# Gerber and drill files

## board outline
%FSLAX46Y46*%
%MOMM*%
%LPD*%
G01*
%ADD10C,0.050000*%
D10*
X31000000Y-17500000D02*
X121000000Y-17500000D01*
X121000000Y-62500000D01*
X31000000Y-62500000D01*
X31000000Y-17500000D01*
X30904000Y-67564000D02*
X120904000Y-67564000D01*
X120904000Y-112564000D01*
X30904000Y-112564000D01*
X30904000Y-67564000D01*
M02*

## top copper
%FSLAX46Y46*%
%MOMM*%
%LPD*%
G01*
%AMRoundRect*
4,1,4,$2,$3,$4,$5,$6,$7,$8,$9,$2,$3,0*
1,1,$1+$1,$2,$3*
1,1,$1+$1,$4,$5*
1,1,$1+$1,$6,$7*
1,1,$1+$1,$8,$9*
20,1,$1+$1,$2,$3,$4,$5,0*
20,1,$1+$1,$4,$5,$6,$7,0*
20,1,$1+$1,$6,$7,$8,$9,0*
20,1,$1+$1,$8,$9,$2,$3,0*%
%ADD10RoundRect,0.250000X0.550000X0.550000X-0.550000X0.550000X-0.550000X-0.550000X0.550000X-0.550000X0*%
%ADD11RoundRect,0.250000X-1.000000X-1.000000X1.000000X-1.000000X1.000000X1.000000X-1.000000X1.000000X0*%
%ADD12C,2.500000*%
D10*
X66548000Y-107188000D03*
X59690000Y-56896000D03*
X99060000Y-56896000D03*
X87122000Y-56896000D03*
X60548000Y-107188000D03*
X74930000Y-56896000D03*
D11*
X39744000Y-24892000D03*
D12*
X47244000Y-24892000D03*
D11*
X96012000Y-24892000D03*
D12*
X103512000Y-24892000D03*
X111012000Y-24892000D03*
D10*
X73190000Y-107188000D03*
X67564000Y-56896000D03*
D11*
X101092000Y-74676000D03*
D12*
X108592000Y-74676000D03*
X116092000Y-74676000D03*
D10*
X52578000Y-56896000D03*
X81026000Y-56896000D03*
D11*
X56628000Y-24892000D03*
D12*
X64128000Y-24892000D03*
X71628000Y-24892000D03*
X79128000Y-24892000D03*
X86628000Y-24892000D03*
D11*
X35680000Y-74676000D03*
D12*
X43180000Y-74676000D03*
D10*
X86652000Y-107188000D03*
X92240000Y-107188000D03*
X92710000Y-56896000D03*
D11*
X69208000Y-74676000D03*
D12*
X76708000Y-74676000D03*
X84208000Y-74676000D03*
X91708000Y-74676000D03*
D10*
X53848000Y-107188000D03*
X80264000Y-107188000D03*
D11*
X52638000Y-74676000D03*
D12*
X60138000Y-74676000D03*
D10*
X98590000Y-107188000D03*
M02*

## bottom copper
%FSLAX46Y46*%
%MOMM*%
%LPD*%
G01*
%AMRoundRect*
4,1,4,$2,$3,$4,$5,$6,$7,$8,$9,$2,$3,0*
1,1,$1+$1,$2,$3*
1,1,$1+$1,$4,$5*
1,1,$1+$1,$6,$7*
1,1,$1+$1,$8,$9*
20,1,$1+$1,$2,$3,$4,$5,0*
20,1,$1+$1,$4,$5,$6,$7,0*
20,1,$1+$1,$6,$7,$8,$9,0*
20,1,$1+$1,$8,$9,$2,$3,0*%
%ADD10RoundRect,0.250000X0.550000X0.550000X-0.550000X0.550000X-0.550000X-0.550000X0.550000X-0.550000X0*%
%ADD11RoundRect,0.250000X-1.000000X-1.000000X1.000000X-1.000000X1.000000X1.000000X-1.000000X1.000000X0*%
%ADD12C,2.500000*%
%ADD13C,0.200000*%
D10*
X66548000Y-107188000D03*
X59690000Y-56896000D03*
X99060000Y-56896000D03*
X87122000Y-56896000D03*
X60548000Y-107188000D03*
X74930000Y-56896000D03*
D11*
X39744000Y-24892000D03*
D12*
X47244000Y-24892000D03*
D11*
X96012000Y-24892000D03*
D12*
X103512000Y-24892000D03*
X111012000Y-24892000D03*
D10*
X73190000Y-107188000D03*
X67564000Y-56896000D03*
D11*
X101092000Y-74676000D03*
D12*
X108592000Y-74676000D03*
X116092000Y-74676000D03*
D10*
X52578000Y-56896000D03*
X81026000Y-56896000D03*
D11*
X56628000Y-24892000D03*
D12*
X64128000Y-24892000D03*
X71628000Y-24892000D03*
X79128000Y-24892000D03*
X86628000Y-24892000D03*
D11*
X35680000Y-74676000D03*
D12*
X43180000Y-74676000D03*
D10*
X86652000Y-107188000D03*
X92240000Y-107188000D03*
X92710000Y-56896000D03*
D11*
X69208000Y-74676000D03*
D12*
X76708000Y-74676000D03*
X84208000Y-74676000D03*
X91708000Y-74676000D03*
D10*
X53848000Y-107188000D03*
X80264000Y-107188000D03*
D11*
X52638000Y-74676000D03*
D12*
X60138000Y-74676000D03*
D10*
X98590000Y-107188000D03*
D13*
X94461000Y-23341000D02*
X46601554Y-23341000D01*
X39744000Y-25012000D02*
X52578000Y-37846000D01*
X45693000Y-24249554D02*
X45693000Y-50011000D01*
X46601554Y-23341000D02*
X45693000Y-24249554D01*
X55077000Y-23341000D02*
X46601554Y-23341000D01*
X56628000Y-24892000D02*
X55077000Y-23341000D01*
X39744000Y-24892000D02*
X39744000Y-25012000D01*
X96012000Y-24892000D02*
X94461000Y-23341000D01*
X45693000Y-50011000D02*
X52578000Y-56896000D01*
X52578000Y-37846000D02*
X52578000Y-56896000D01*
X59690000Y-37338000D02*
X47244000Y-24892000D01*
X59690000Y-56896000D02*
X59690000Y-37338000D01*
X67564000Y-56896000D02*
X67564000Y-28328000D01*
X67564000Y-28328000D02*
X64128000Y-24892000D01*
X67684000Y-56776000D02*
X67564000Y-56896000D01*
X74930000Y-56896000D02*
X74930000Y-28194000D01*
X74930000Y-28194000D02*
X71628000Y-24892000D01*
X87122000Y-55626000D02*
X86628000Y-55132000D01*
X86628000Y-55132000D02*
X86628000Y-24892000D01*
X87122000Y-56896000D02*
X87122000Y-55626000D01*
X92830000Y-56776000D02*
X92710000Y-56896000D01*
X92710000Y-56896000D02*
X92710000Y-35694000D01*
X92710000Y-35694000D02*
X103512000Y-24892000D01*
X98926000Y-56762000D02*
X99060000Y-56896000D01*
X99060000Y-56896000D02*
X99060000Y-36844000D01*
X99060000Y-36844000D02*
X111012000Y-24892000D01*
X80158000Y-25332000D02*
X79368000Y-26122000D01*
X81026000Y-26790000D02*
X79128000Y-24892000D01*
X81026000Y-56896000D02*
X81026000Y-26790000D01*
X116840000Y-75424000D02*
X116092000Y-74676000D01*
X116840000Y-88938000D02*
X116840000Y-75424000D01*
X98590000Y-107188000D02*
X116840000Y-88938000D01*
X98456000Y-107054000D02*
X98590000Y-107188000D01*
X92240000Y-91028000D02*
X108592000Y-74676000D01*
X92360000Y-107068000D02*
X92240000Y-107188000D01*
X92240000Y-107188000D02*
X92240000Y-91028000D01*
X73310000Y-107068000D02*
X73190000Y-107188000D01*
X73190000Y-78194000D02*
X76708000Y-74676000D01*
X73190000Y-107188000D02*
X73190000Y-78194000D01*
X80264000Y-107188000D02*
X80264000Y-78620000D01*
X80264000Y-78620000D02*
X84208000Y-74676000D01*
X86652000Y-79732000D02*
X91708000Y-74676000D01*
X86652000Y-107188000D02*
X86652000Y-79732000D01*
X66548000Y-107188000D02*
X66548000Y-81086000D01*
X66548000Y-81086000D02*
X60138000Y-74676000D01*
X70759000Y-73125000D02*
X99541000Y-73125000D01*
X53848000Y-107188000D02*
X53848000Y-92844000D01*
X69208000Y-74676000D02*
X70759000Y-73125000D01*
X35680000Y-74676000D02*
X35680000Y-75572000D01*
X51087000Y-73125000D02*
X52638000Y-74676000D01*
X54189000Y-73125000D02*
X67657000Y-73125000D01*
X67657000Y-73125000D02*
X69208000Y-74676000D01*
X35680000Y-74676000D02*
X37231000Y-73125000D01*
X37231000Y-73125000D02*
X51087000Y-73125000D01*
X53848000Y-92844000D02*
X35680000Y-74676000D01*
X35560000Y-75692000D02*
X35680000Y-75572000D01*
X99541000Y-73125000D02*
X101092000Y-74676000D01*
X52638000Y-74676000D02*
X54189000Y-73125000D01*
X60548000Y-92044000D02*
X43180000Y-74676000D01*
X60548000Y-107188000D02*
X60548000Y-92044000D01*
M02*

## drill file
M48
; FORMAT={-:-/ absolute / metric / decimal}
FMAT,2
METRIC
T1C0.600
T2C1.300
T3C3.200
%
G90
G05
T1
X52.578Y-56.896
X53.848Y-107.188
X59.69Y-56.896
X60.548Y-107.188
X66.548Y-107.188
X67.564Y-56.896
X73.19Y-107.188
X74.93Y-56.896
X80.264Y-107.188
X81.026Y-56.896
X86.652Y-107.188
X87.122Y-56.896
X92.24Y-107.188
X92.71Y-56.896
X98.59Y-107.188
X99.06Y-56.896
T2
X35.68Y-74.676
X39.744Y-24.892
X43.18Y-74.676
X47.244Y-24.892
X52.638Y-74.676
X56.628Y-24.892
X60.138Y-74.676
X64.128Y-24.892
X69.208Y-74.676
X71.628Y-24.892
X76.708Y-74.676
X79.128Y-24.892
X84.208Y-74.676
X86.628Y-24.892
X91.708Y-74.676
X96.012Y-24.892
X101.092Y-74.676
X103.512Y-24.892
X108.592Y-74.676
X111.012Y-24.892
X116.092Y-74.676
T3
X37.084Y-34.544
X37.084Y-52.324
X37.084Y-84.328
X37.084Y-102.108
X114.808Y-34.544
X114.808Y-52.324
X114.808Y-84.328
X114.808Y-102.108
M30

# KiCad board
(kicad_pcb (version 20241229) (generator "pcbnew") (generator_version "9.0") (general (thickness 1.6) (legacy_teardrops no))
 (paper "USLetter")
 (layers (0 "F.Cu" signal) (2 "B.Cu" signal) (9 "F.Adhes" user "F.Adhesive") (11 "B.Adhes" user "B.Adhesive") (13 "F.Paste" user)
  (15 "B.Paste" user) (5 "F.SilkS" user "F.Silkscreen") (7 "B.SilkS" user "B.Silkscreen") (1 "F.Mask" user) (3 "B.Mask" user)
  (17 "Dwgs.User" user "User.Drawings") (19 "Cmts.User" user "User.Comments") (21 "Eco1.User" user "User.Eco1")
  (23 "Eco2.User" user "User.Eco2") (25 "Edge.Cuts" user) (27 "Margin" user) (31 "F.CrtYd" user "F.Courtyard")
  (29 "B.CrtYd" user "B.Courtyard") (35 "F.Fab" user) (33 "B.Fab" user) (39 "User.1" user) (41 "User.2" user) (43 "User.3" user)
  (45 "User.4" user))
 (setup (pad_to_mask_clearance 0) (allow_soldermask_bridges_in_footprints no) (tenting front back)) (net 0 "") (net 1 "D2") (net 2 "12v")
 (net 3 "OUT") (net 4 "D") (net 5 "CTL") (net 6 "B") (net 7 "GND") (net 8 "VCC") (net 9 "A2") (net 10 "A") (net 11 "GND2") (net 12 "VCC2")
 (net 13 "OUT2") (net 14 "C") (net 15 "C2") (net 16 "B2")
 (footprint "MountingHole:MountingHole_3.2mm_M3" (layer "F.Cu") (at 114.808 102.108)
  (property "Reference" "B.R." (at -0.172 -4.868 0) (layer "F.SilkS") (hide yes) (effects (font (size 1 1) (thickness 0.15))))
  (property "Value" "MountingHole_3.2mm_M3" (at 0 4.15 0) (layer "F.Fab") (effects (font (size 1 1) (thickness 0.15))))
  (pad "" np_thru_hole circle (at 0 0) (size 3.2 3.2) (drill 3.2) (layers "*.Cu" "*.Mask")))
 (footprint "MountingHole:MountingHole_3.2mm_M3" (layer "F.Cu") (at 114.808 52.324)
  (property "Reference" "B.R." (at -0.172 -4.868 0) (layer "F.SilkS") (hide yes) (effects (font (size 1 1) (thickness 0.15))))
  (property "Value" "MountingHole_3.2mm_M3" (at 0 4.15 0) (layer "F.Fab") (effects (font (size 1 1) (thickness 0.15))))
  (pad "" np_thru_hole circle (at 0 0) (size 3.2 3.2) (drill 3.2) (layers "*.Cu" "*.Mask")))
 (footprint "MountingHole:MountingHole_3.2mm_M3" (layer "F.Cu") (at 37.084 102.108)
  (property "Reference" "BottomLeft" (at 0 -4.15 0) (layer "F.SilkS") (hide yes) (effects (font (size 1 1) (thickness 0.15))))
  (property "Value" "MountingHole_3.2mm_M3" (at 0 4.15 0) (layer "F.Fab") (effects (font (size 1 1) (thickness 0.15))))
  (pad "" np_thru_hole circle (at 0 0) (size 3.2 3.2) (drill 3.2) (layers "*.Cu" "*.Mask")))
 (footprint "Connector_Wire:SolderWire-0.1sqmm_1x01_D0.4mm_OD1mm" (layer "F.Cu") (at 66.548 107.188 180)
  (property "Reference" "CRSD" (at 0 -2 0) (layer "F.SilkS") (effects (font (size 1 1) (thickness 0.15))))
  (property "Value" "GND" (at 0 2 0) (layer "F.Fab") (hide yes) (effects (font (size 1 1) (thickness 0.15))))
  (pad "1" thru_hole roundrect (at 0 0 180) (size 1.6 1.6) (drill 0.6) (layers "*.Cu" "*.Mask") (remove_unused_layers no)
   (roundrect_rratio 0.15625) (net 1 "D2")))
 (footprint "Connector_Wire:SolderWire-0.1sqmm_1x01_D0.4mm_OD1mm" (layer "F.Cu") (at 59.69 56.896 180)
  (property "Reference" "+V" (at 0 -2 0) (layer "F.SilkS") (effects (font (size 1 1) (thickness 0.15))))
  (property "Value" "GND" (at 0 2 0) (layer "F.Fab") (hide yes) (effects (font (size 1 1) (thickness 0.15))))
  (pad "1" thru_hole roundrect (at 0 0 180) (size 1.6 1.6) (drill 0.6) (layers "*.Cu" "*.Mask") (remove_unused_layers no)
   (roundrect_rratio 0.15625) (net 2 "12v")))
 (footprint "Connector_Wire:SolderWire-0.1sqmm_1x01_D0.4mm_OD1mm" (layer "F.Cu") (at 99.06 56.896 180)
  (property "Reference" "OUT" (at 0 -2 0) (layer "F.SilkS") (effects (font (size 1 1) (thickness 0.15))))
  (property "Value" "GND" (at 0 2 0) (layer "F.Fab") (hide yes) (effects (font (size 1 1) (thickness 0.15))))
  (pad "1" thru_hole roundrect (at 0 0 180) (size 1.6 1.6) (drill 0.6) (layers "*.Cu" "*.Mask") (remove_unused_layers no)
   (roundrect_rratio 0.15625) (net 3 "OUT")))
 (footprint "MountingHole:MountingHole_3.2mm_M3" (layer "F.Cu") (at 114.808 84.328)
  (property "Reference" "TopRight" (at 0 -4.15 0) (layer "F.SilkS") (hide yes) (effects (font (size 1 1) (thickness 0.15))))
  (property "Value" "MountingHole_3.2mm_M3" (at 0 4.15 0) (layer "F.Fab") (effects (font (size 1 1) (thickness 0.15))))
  (pad "" np_thru_hole circle (at 0 0) (size 3.2 3.2) (drill 3.2) (layers "*.Cu" "*.Mask")))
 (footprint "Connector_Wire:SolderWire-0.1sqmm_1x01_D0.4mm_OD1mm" (layer "F.Cu") (at 87.122 56.896 180)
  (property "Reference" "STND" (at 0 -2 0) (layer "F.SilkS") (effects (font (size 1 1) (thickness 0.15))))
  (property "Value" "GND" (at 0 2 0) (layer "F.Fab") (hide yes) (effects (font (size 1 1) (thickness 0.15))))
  (pad "1" thru_hole roundrect (at 0 0 180) (size 1.6 1.6) (drill 0.6) (layers "*.Cu" "*.Mask") (remove_unused_layers no)
   (roundrect_rratio 0.15625) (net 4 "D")))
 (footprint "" (layer "F.Cu") (at 60.548 107.188)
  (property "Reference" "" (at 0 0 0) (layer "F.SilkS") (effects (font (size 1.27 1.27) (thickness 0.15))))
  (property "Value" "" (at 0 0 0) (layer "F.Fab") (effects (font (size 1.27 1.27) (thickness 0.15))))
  (pad "1" thru_hole roundrect (at 0 0 180) (size 1.6 1.6) (drill 0.6) (layers "*.Cu" "*.Mask") (remove_unused_layers no)
   (roundrect_rratio 0.15625) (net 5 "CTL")))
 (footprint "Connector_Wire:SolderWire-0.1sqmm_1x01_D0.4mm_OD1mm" (layer "F.Cu") (at 74.93 56.896 180)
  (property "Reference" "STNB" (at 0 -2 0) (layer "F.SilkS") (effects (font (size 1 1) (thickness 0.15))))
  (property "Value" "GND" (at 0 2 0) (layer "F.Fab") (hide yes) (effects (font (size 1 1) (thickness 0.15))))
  (pad "1" thru_hole roundrect (at 0 0 180) (size 1.6 1.6) (drill 0.6) (layers "*.Cu" "*.Mask") (remove_unused_layers no)
   (roundrect_rratio 0.15625) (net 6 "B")))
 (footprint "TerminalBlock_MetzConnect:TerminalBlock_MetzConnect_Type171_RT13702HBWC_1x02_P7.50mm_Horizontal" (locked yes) (layer "F.Cu")
  (at 39.744 24.892)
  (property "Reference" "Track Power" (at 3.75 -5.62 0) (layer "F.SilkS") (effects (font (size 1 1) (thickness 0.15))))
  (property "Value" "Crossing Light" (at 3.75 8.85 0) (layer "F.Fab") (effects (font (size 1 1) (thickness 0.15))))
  (pad "1" thru_hole roundrect (at 0 0) (size 2.5 2.5) (drill 1.3) (layers "*.Cu" "*.Mask") (remove_unused_layers no) (roundrect_rratio 0.1)
   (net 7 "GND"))
  (pad "2" thru_hole circle (at 7.5 0) (size 2.5 2.5) (drill 1.3) (layers "*.Cu" "*.Mask") (remove_unused_layers no) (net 2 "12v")))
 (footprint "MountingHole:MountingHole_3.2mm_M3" (layer "F.Cu") (at 37.084 34.544)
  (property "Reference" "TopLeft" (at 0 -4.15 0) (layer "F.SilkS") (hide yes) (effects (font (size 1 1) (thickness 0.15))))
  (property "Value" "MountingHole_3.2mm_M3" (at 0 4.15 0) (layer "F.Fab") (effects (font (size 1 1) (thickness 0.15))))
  (pad "" np_thru_hole circle (at 0 0) (size 3.2 3.2) (drill 3.2) (layers "*.Cu" "*.Mask")))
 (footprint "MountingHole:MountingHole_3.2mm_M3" (layer "F.Cu") (at 37.084 52.324)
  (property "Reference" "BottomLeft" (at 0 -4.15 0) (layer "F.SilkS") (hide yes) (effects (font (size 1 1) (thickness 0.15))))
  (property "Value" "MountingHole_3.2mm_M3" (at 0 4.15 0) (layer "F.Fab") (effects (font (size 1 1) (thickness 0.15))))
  (pad "" np_thru_hole circle (at 0 0) (size 3.2 3.2) (drill 3.2) (layers "*.Cu" "*.Mask")))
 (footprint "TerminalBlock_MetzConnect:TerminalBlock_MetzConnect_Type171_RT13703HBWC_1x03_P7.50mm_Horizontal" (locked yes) (layer "F.Cu")
  (at 96.012 24.892)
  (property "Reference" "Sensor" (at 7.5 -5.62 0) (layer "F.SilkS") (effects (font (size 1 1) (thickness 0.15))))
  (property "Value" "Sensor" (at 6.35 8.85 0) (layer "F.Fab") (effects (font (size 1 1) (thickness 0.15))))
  (pad "1" thru_hole roundrect (at 0 0) (size 2.5 2.5) (drill 1.3) (layers "*.Cu" "*.Mask") (remove_unused_layers no) (roundrect_rratio 0.1)
   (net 7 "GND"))
  (pad "2" thru_hole circle (at 7.5 0) (size 2.5 2.5) (drill 1.3) (layers "*.Cu" "*.Mask") (remove_unused_layers no) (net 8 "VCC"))
  (pad "3" thru_hole circle (at 15 0) (size 2.5 2.5) (drill 1.3) (layers "*.Cu" "*.Mask") (remove_unused_layers no) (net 3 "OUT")))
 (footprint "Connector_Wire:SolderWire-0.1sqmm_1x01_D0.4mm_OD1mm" (layer "F.Cu") (at 73.19 107.188 180)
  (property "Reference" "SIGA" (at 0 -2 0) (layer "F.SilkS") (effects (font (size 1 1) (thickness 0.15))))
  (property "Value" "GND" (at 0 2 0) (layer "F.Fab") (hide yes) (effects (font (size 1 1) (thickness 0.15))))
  (pad "1" thru_hole roundrect (at 0 0 180) (size 1.6 1.6) (drill 0.6) (layers "*.Cu" "*.Mask") (remove_unused_layers no)
   (roundrect_rratio 0.15625) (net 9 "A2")))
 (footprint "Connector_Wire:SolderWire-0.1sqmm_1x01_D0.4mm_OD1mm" (layer "F.Cu") (at 67.564 56.896 180)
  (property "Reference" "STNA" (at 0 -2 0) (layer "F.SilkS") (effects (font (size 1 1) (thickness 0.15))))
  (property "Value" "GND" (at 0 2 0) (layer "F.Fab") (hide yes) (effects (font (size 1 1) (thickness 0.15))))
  (pad "1" thru_hole roundrect (at 0 0 180) (size 1.6 1.6) (drill 0.6) (layers "*.Cu" "*.Mask") (remove_unused_layers no)
   (roundrect_rratio 0.15625) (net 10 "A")))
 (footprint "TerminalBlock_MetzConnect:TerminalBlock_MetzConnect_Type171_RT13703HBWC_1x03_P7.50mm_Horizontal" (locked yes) (layer "F.Cu")
  (at 101.092 74.676)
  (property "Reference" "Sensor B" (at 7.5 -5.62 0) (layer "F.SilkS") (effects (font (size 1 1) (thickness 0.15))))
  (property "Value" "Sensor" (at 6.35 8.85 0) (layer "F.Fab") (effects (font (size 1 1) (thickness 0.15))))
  (pad "1" thru_hole roundrect (at 0 0) (size 2.5 2.5) (drill 1.3) (layers "*.Cu" "*.Mask") (remove_unused_layers no) (roundrect_rratio 0.1)
   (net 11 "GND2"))
  (pad "2" thru_hole circle (at 7.5 0) (size 2.5 2.5) (drill 1.3) (layers "*.Cu" "*.Mask") (remove_unused_layers no) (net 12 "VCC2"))
  (pad "3" thru_hole circle (at 15 0) (size 2.5 2.5) (drill 1.3) (layers "*.Cu" "*.Mask") (remove_unused_layers no) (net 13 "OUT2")))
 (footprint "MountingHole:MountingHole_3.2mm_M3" (layer "F.Cu") (at 114.808 34.544)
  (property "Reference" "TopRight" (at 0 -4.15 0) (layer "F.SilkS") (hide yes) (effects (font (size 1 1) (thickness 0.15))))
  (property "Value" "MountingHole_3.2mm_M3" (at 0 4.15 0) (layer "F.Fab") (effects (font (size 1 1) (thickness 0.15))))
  (pad "" np_thru_hole circle (at 0 0) (size 3.2 3.2) (drill 3.2) (layers "*.Cu" "*.Mask")))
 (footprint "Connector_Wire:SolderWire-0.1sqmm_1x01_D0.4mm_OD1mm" (layer "F.Cu") (at 52.578 56.896 180)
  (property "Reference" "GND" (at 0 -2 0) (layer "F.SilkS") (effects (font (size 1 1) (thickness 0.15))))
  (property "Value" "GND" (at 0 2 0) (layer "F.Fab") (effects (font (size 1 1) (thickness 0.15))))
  (pad "1" thru_hole roundrect (at 0 0 180) (size 1.6 1.6) (drill 0.6) (layers "*.Cu" "*.Mask") (remove_unused_layers no)
   (roundrect_rratio 0.15625) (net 7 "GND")))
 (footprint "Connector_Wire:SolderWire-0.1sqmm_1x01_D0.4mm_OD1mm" (layer "F.Cu") (at 81.026 56.896 180)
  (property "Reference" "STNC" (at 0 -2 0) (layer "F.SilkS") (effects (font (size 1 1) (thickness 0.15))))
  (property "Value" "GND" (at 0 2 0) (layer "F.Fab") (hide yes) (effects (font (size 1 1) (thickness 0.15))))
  (pad "1" thru_hole roundrect (at 0 0 180) (size 1.6 1.6) (drill 0.6) (layers "*.Cu" "*.Mask") (remove_unused_layers no)
   (roundrect_rratio 0.15625) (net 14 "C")))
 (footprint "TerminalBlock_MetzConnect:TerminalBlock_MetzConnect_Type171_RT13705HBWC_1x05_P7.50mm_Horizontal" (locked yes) (layer "F.Cu")
  (at 56.628 24.892)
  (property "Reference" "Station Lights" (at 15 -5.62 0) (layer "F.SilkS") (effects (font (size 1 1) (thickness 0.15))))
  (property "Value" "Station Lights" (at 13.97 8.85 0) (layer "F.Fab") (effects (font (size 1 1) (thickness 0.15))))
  (pad "1" thru_hole roundrect (at 0 0) (size 2.5 2.5) (drill 1.3) (layers "*.Cu" "*.Mask") (remove_unused_layers no) (roundrect_rratio 0.1)
   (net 7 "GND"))
  (pad "2" thru_hole circle (at 7.5 0) (size 2.5 2.5) (drill 1.3) (layers "*.Cu" "*.Mask") (remove_unused_layers no) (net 10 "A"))
  (pad "3" thru_hole circle (at 15 0) (size 2.5 2.5) (drill 1.3) (layers "*.Cu" "*.Mask") (remove_unused_layers no) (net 6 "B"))
  (pad "4" thru_hole circle (at 22.5 0) (size 2.5 2.5) (drill 1.3) (layers "*.Cu" "*.Mask") (remove_unused_layers no) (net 14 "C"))
  (pad "5" thru_hole circle (at 30 0) (size 2.5 2.5) (drill 1.3) (layers "*.Cu" "*.Mask") (remove_unused_layers no) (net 4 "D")))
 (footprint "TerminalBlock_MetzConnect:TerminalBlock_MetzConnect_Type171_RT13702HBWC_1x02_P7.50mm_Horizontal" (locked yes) (layer "F.Cu")
  (at 35.68 74.676)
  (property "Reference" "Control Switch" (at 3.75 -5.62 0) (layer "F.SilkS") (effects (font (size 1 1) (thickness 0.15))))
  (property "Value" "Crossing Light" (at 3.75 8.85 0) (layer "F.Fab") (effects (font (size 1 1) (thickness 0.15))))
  (pad "1" thru_hole roundrect (at 0 0) (size 2.5 2.5) (drill 1.3) (layers "*.Cu" "*.Mask") (remove_unused_layers no) (roundrect_rratio 0.1)
   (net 11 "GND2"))
  (pad "2" thru_hole circle (at 7.5 0) (size 2.5 2.5) (drill 1.3) (layers "*.Cu" "*.Mask") (remove_unused_layers no) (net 5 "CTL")))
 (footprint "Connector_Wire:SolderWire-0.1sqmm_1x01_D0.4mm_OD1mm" (layer "F.Cu") (at 86.652 107.188 180)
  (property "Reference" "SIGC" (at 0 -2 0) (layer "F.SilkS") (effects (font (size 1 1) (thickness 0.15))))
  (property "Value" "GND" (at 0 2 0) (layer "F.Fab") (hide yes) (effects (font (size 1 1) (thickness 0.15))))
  (pad "1" thru_hole roundrect (at 0 0 180) (size 1.6 1.6) (drill 0.6) (layers "*.Cu" "*.Mask") (remove_unused_layers no)
   (roundrect_rratio 0.15625) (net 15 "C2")))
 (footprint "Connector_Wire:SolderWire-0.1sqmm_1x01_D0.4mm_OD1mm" (layer "F.Cu") (at 92.24 107.188 180)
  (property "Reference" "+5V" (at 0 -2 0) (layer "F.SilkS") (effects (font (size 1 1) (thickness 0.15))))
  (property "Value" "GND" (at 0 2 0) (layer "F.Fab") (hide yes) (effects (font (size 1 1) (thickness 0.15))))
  (pad "1" thru_hole roundrect (at 0 0 180) (size 1.6 1.6) (drill 0.6) (layers "*.Cu" "*.Mask") (remove_unused_layers no)
   (roundrect_rratio 0.15625) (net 12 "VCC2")))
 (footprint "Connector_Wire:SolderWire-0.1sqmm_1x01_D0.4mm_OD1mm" (layer "F.Cu") (at 92.71 56.896 180)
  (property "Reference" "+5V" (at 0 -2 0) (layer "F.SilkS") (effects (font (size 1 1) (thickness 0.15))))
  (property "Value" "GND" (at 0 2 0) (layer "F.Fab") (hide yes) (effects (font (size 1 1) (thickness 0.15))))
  (pad "1" thru_hole roundrect (at 0 0 180) (size 1.6 1.6) (drill 0.6) (layers "*.Cu" "*.Mask") (remove_unused_layers no)
   (roundrect_rratio 0.15625) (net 8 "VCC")))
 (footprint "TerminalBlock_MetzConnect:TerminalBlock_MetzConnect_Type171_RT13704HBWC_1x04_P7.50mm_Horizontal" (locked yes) (layer "F.Cu")
  (at 69.208 74.676)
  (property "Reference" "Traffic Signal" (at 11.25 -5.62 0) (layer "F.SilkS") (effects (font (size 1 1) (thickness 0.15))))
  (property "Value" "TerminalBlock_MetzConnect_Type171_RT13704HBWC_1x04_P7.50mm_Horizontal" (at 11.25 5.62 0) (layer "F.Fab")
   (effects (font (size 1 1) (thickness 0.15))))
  (pad "1" thru_hole roundrect (at 0 0) (size 2.5 2.5) (drill 1.3) (layers "*.Cu" "*.Mask") (remove_unused_layers no) (roundrect_rratio 0.1)
   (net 11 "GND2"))
  (pad "2" thru_hole circle (at 7.5 0) (size 2.5 2.5) (drill 1.3) (layers "*.Cu" "*.Mask") (remove_unused_layers no) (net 9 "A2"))
  (pad "3" thru_hole circle (at 15 0) (size 2.5 2.5) (drill 1.3) (layers "*.Cu" "*.Mask") (remove_unused_layers no) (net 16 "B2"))
  (pad "4" thru_hole circle (at 22.5 0) (size 2.5 2.5) (drill 1.3) (layers "*.Cu" "*.Mask") (remove_unused_layers no) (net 15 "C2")))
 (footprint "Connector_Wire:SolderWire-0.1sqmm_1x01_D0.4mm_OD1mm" (layer "F.Cu") (at 53.848 107.188 180)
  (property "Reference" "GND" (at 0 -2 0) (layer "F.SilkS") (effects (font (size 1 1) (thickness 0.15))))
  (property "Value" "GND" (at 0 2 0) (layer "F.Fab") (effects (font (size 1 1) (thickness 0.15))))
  (pad "1" thru_hole roundrect (at 0 0 180) (size 1.6 1.6) (drill 0.6) (layers "*.Cu" "*.Mask") (remove_unused_layers no)
   (roundrect_rratio 0.15625) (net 11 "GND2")))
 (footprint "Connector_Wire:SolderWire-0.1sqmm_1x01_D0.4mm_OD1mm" (layer "F.Cu") (at 80.264 107.188 180)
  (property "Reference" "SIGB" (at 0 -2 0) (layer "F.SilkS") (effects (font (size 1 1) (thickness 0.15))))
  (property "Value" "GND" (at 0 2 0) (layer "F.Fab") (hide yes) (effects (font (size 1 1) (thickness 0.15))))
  (pad "1" thru_hole roundrect (at 0 0 180) (size 1.6 1.6) (drill 0.6) (layers "*.Cu" "*.Mask") (remove_unused_layers no)
   (roundrect_rratio 0.15625) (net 16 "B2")))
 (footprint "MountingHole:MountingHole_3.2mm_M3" (layer "F.Cu") (at 37.084 84.328)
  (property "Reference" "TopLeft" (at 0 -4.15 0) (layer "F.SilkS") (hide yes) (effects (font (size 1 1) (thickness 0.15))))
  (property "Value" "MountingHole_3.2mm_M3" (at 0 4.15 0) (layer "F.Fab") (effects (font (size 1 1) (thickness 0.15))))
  (pad "" np_thru_hole circle (at 0 0) (size 3.2 3.2) (drill 3.2) (layers "*.Cu" "*.Mask")))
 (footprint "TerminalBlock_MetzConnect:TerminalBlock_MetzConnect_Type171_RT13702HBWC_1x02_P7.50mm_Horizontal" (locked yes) (layer "F.Cu")
  (at 52.638 74.676)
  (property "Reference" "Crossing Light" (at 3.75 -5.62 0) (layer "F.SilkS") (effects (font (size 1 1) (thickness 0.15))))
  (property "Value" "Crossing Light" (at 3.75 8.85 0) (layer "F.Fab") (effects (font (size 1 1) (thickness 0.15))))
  (pad "1" thru_hole roundrect (at 0 0) (size 2.5 2.5) (drill 1.3) (layers "*.Cu" "*.Mask") (remove_unused_layers no) (roundrect_rratio 0.1)
   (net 11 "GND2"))
  (pad "2" thru_hole circle (at 7.5 0) (size 2.5 2.5) (drill 1.3) (layers "*.Cu" "*.Mask") (remove_unused_layers no) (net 1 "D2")))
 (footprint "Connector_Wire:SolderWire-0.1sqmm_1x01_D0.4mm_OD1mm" (layer "F.Cu") (at 98.59 107.188 180)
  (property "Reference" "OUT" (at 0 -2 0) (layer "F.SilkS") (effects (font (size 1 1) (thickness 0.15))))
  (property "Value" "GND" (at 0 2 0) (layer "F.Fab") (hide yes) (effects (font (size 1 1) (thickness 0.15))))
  (pad "1" thru_hole roundrect (at 0 0 180) (size 1.6 1.6) (drill 0.6) (layers "*.Cu" "*.Mask") (remove_unused_layers no)
   (roundrect_rratio 0.15625) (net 13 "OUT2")))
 (gr_rect (start 31 17.5) (end 121 62.5) (stroke (width 0.05) (type solid)) (fill no) (layer "Edge.Cuts"))
 (gr_rect (start 30.904 67.564) (end 120.904 112.564) (stroke (width 0.05) (type solid)) (fill no) (layer "Edge.Cuts"))
 (segment (start 94.461 23.341) (end 46.601554 23.341) (width 0.2) (layer "B.Cu") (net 7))
 (segment (start 39.744 25.012) (end 52.578 37.846) (width 0.2) (layer "B.Cu") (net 7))
 (segment (start 45.693 24.249554) (end 45.693 50.011) (width 0.2) (layer "B.Cu") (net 7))
 (segment (start 46.601554 23.341) (end 45.693 24.249554) (width 0.2) (layer "B.Cu") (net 7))
 (segment (start 55.077 23.341) (end 46.601554 23.341) (width 0.2) (layer "B.Cu") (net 7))
 (segment (start 56.628 24.892) (end 55.077 23.341) (width 0.2) (layer "B.Cu") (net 7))
 (segment (start 39.744 24.892) (end 39.744 25.012) (width 0.2) (layer "B.Cu") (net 7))
 (segment (start 96.012 24.892) (end 94.461 23.341) (width 0.2) (layer "B.Cu") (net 7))
 (segment (start 45.693 50.011) (end 52.578 56.896) (width 0.2) (layer "B.Cu") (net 7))
 (segment (start 52.578 37.846) (end 52.578 56.896) (width 0.2) (layer "B.Cu") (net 7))
 (segment (start 59.69 37.338) (end 47.244 24.892) (width 0.2) (layer "B.Cu") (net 2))
 (segment (start 59.69 56.896) (end 59.69 37.338) (width 0.2) (layer "B.Cu") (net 2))
 (segment (start 67.564 56.896) (end 67.564 28.328) (width 0.2) (layer "B.Cu") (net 10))
 (segment (start 67.564 28.328) (end 64.128 24.892) (width 0.2) (layer "B.Cu") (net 10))
 (segment (start 67.684 56.776) (end 67.564 56.896) (width 0.2) (layer "B.Cu") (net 10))
 (segment (start 74.93 56.896) (end 74.93 28.194) (width 0.2) (layer "B.Cu") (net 6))
 (segment (start 74.93 28.194) (end 71.628 24.892) (width 0.2) (layer "B.Cu") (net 6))
 (segment (start 87.122 55.626) (end 86.628 55.132) (width 0.2) (layer "B.Cu") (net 4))
 (segment (start 86.628 55.132) (end 86.628 24.892) (width 0.2) (layer "B.Cu") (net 4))
 (segment (start 87.122 56.896) (end 87.122 55.626) (width 0.2) (layer "B.Cu") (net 4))
 (segment (start 92.83 56.776) (end 92.71 56.896) (width 0.2) (layer "B.Cu") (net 8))
 (segment (start 92.71 56.896) (end 92.71 35.694) (width 0.2) (layer "B.Cu") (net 8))
 (segment (start 92.71 35.694) (end 103.512 24.892) (width 0.2) (layer "B.Cu") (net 8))
 (segment (start 98.926 56.762) (end 99.06 56.896) (width 0.2) (layer "B.Cu") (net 3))
 (segment (start 99.06 56.896) (end 99.06 36.844) (width 0.2) (layer "B.Cu") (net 3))
 (segment (start 99.06 36.844) (end 111.012 24.892) (width 0.2) (layer "B.Cu") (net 3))
 (segment (start 80.158 25.332) (end 79.368 26.122) (width 0.2) (layer "B.Cu") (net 14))
 (segment (start 81.026 26.79) (end 79.128 24.892) (width 0.2) (layer "B.Cu") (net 14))
 (segment (start 81.026 56.896) (end 81.026 26.79) (width 0.2) (layer "B.Cu") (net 14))
 (segment (start 116.84 75.424) (end 116.092 74.676) (width 0.2) (layer "B.Cu") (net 13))
 (segment (start 116.84 88.938) (end 116.84 75.424) (width 0.2) (layer "B.Cu") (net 13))
 (segment (start 98.59 107.188) (end 116.84 88.938) (width 0.2) (layer "B.Cu") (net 13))
 (segment (start 98.456 107.054) (end 98.59 107.188) (width 0.2) (layer "B.Cu") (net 13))
 (segment (start 92.24 91.028) (end 108.592 74.676) (width 0.2) (layer "B.Cu") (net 12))
 (segment (start 92.36 107.068) (end 92.24 107.188) (width 0.2) (layer "B.Cu") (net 12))
 (segment (start 92.24 107.188) (end 92.24 91.028) (width 0.2) (layer "B.Cu") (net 12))
 (segment (start 73.31 107.068) (end 73.19 107.188) (width 0.2) (layer "B.Cu") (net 9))
 (segment (start 73.19 78.194) (end 76.708 74.676) (width 0.2) (layer "B.Cu") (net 9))
 (segment (start 73.19 107.188) (end 73.19 78.194) (width 0.2) (layer "B.Cu") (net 9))
 (segment (start 80.264 107.188) (end 80.264 78.62) (width 0.2) (layer "B.Cu") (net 16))
 (segment (start 80.264 78.62) (end 84.208 74.676) (width 0.2) (layer "B.Cu") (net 16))
 (segment (start 86.652 79.732) (end 91.708 74.676) (width 0.2) (layer "B.Cu") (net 15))
 (segment (start 86.652 107.188) (end 86.652 79.732) (width 0.2) (layer "B.Cu") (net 15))
 (segment (start 66.548 107.188) (end 66.548 81.086) (width 0.2) (layer "B.Cu") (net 1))
 (segment (start 66.548 81.086) (end 60.138 74.676) (width 0.2) (layer "B.Cu") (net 1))
 (segment (start 70.759 73.125) (end 99.541 73.125) (width 0.2) (layer "B.Cu") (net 11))
 (segment (start 53.848 107.188) (end 53.848 92.844) (width 0.2) (layer "B.Cu") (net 11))
 (segment (start 69.208 74.676) (end 70.759 73.125) (width 0.2) (layer "B.Cu") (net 11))
 (segment (start 35.68 74.676) (end 35.68 75.572) (width 0.2) (layer "B.Cu") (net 11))
 (segment (start 51.087 73.125) (end 52.638 74.676) (width 0.2) (layer "B.Cu") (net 11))
 (segment (start 54.189 73.125) (end 67.657 73.125) (width 0.2) (layer "B.Cu") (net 11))
 (segment (start 67.657 73.125) (end 69.208 74.676) (width 0.2) (layer "B.Cu") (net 11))
 (segment (start 35.68 74.676) (end 37.231 73.125) (width 0.2) (layer "B.Cu") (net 11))
 (segment (start 37.231 73.125) (end 51.087 73.125) (width 0.2) (layer "B.Cu") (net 11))
 (segment (start 53.848 92.844) (end 35.68 74.676) (width 0.2) (layer "B.Cu") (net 11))
 (segment (start 35.56 75.692) (end 35.68 75.572) (width 0.2) (layer "B.Cu") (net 11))
 (segment (start 99.541 73.125) (end 101.092 74.676) (width 0.2) (layer "B.Cu") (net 11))
 (segment (start 52.638 74.676) (end 54.189 73.125) (width 0.2) (layer "B.Cu") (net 11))
 (segment (start 60.548 92.044) (end 43.18 74.676) (width 0.2) (layer "B.Cu") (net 5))
 (segment (start 60.548 107.188) (end 60.548 92.044) (width 0.2) (layer "B.Cu") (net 5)))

